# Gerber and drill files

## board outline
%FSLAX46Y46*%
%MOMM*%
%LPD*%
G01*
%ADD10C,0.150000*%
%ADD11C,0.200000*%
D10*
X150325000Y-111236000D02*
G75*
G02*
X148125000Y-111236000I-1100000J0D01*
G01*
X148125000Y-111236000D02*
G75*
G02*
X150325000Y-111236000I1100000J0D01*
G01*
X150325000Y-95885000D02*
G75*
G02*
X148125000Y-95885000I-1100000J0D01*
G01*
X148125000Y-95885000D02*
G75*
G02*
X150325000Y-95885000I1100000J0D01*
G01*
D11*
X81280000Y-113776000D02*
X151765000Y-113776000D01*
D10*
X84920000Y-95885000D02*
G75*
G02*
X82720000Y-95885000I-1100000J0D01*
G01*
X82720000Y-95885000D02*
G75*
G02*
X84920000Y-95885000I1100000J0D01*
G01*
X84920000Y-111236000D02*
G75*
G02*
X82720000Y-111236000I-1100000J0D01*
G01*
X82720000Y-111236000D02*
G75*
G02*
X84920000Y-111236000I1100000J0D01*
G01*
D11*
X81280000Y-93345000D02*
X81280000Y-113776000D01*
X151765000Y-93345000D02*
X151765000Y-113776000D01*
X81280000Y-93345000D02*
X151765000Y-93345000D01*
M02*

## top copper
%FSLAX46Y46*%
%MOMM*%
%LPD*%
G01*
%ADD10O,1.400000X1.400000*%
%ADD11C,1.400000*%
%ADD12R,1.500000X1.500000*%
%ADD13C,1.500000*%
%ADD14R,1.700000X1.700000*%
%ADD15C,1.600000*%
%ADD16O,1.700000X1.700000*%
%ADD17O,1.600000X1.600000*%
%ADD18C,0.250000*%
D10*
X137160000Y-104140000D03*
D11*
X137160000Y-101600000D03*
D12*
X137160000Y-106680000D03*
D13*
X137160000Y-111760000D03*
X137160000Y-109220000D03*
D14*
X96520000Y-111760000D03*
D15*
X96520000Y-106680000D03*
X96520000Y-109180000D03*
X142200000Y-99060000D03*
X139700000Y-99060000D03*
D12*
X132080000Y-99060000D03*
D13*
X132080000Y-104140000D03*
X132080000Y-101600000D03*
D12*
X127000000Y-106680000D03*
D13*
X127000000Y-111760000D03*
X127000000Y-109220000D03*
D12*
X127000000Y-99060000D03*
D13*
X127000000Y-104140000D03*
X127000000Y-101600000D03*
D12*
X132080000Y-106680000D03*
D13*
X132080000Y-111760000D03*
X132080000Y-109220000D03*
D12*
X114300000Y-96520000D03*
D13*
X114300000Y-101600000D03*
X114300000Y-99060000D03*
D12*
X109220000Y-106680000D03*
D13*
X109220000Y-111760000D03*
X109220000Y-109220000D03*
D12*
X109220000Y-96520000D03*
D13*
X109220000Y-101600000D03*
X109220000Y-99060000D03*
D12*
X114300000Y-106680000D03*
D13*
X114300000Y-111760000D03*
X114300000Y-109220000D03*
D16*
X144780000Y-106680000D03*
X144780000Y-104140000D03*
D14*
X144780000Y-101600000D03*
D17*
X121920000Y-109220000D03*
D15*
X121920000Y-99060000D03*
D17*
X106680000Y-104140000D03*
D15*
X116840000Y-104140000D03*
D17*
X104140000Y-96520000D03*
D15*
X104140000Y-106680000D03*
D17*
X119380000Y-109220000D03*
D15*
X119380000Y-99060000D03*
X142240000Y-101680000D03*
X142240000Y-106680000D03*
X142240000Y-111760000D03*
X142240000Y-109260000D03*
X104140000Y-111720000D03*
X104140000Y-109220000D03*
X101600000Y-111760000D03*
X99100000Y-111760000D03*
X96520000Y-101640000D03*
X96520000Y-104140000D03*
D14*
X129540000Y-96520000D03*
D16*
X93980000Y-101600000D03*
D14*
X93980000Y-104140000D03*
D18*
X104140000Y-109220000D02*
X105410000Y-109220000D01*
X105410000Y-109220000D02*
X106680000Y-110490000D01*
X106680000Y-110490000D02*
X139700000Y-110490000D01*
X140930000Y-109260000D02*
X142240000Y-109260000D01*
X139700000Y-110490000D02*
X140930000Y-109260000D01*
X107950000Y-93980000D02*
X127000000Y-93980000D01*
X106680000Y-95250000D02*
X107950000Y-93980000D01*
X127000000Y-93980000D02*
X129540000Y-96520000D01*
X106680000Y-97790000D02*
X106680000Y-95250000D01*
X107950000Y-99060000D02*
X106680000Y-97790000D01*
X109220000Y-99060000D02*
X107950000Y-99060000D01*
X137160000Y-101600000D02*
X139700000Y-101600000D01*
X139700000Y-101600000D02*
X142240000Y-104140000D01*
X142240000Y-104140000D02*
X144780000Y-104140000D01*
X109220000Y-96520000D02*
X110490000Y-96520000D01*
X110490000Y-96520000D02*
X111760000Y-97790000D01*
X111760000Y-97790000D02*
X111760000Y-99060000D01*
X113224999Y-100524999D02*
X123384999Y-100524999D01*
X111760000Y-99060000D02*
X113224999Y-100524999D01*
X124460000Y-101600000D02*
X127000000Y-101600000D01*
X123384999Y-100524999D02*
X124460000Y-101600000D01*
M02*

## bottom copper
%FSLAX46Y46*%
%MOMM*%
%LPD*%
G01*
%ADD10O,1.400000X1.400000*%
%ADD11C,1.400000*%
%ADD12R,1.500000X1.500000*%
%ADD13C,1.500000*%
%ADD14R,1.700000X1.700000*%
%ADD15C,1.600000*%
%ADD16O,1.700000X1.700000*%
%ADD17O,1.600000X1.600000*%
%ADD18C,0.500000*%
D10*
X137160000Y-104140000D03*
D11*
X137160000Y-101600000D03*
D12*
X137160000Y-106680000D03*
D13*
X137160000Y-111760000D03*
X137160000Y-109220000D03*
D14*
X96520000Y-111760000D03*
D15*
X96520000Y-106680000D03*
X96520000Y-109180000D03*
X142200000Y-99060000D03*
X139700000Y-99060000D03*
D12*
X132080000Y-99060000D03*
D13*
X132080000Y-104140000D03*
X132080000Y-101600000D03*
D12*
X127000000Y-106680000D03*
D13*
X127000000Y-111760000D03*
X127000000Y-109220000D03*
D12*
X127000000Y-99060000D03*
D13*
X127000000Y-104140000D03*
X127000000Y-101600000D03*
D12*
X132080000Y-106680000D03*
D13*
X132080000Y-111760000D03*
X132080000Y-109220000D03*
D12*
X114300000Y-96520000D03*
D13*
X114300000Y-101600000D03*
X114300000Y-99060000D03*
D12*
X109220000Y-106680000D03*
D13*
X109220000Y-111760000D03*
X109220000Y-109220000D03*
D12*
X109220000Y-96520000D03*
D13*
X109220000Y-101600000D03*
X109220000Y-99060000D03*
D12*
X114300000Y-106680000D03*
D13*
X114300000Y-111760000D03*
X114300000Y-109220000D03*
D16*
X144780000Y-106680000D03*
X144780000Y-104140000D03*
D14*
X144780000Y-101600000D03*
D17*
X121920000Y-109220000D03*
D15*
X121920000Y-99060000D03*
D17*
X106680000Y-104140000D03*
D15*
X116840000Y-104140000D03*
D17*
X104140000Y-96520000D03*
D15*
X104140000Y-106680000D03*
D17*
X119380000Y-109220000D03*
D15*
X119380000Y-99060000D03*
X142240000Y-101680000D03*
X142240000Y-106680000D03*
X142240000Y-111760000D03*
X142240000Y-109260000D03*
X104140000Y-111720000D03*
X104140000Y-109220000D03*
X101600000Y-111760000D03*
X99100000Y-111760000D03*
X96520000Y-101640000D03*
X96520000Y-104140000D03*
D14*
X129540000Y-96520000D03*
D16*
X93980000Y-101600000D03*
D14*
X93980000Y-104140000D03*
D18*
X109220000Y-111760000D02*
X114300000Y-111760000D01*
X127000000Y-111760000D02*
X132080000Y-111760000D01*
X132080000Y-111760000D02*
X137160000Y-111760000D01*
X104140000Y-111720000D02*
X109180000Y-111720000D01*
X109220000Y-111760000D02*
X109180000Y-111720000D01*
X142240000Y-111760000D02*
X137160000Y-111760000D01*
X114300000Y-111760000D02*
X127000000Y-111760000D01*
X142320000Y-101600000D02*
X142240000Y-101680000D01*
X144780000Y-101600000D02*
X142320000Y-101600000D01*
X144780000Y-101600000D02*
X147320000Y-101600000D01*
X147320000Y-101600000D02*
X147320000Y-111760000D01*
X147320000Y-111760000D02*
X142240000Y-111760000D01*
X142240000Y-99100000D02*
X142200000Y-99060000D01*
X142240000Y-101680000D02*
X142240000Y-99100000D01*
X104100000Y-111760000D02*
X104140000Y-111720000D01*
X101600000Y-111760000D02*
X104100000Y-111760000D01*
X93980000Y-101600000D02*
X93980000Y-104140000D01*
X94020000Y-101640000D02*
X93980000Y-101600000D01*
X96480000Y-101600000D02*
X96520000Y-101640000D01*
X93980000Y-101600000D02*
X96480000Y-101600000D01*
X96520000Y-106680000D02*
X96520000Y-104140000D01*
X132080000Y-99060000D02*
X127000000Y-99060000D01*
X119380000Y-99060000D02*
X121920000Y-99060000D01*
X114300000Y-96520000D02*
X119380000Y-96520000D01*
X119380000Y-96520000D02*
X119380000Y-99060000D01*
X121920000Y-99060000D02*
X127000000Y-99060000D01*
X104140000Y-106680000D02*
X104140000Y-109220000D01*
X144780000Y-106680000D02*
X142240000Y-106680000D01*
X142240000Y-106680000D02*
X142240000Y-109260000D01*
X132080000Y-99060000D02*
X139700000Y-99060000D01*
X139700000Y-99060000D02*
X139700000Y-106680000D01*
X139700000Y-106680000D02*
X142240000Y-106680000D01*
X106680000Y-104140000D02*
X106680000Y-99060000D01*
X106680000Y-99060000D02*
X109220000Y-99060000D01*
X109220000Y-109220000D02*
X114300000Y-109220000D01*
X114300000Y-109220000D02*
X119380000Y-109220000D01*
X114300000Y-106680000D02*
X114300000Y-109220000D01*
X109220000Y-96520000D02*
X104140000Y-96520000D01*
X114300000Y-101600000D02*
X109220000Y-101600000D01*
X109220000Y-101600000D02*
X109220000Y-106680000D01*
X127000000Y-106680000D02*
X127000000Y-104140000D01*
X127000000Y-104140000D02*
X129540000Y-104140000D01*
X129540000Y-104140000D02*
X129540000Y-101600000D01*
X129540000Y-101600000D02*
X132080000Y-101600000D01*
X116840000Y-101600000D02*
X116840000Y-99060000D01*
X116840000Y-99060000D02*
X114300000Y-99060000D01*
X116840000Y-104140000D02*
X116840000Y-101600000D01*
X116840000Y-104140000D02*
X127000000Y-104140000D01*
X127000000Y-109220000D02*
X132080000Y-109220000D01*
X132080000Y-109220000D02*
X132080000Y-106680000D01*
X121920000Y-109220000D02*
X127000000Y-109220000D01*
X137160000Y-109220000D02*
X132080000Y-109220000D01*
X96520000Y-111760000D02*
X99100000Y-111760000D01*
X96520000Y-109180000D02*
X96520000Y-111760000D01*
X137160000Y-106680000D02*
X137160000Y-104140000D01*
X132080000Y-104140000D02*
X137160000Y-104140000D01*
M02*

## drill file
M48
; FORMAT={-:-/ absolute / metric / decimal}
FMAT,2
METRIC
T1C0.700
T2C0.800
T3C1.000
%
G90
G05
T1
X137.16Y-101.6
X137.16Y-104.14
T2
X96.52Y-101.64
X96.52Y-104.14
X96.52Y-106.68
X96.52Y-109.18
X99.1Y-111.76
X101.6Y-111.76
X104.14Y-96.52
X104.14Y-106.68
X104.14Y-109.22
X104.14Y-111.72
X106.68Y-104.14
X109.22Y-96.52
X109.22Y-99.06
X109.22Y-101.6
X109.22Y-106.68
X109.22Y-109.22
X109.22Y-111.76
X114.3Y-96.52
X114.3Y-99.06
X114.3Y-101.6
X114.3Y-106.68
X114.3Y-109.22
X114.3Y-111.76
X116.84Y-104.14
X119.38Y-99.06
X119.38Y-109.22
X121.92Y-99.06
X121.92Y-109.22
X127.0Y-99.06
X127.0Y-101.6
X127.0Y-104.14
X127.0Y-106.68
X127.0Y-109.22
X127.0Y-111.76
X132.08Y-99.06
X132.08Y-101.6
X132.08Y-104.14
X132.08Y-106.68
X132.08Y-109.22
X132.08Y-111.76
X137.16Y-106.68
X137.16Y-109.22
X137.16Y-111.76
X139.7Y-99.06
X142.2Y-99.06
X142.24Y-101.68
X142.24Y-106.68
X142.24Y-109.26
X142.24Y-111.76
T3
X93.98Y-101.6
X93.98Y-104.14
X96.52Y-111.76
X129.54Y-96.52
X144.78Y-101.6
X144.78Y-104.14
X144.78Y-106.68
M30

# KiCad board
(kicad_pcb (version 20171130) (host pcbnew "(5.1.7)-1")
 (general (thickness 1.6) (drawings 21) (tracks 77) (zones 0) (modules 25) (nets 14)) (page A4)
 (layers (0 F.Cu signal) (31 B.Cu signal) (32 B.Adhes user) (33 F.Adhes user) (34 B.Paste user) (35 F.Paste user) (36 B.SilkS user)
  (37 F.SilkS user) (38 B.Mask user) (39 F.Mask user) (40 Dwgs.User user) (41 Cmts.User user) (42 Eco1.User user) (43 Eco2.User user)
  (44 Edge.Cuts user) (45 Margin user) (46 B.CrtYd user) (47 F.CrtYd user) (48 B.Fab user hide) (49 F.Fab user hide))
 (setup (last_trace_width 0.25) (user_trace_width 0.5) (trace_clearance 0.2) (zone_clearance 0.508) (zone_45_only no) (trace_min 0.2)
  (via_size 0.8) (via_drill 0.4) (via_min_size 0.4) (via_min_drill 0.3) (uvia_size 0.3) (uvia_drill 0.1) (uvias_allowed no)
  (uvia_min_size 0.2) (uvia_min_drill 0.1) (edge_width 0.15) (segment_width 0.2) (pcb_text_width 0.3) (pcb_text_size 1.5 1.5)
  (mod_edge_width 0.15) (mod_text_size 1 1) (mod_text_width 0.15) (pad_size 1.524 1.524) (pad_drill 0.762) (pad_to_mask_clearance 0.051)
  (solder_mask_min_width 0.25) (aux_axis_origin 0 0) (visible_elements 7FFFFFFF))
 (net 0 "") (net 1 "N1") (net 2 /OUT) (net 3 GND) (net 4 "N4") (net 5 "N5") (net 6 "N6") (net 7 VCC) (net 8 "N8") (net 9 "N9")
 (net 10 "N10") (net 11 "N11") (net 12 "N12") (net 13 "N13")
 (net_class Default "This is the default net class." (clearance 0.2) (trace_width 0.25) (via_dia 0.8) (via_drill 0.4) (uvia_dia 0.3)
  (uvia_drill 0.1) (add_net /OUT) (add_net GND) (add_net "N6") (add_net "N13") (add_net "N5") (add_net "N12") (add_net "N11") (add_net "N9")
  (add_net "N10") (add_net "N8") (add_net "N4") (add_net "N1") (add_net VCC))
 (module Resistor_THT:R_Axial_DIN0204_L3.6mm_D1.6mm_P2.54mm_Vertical (layer F.Cu) (at 137.16 101.6 270)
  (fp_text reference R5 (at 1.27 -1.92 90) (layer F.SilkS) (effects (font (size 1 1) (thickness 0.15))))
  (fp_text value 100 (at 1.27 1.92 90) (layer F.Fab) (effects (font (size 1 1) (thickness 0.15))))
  (pad 2 thru_hole oval (at 2.54 0 270) (size 1.4 1.4) (drill 0.7) (layers *.Cu *.Mask) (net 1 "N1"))
  (pad 1 thru_hole circle (at 0 0 270) (size 1.4 1.4) (drill 0.7) (layers *.Cu *.Mask) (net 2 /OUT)))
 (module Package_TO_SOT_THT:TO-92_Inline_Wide (layer F.Cu) (at 137.16 106.68 270)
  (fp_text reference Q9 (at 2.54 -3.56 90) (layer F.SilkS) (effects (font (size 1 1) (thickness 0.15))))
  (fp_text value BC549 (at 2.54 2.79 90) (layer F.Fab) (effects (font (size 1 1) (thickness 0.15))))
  (pad 1 thru_hole rect (at 0 0 270) (size 1.5 1.5) (drill 0.8) (layers *.Cu *.Mask) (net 1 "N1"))
  (pad 3 thru_hole circle (at 5.08 0 270) (size 1.5 1.5) (drill 0.8) (layers *.Cu *.Mask) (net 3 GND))
  (pad 2 thru_hole circle (at 2.54 0 270) (size 1.5 1.5) (drill 0.8) (layers *.Cu *.Mask) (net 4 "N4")))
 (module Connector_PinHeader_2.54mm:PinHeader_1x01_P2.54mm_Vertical (layer F.Cu) (at 96.52 111.76)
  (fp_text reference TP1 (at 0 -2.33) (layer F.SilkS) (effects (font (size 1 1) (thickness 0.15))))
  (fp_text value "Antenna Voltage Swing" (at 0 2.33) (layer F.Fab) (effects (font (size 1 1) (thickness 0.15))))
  (pad 1 thru_hole rect (at 0 0) (size 1.7 1.7) (drill 1) (layers *.Cu *.Mask) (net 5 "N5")))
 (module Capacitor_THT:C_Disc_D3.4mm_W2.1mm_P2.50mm (layer F.Cu) (at 96.52 109.18 90)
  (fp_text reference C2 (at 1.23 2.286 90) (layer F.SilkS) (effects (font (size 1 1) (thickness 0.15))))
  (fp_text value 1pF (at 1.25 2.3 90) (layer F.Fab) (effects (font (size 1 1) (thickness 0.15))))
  (pad 2 thru_hole circle (at 2.5 0 90) (size 1.6 1.6) (drill 0.8) (layers *.Cu *.Mask) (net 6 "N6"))
  (pad 1 thru_hole circle (at 0 0 90) (size 1.6 1.6) (drill 0.8) (layers *.Cu *.Mask) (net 5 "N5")))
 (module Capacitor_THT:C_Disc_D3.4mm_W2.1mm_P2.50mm (layer F.Cu) (at 139.7 99.06)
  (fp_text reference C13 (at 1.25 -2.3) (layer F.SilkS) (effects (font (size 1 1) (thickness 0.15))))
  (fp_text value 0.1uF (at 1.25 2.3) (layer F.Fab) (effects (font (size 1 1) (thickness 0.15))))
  (pad 2 thru_hole circle (at 2.5 0) (size 1.6 1.6) (drill 0.8) (layers *.Cu *.Mask) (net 3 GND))
  (pad 1 thru_hole circle (at 0 0) (size 1.6 1.6) (drill 0.8) (layers *.Cu *.Mask) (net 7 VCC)))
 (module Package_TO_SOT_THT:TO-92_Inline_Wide (layer F.Cu) (at 132.08 99.06 270)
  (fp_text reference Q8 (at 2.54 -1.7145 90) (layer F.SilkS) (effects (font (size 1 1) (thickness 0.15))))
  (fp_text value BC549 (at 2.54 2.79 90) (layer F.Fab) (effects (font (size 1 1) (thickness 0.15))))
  (pad 1 thru_hole rect (at 0 0 270) (size 1.5 1.5) (drill 0.8) (layers *.Cu *.Mask) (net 7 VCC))
  (pad 3 thru_hole circle (at 5.08 0 270) (size 1.5 1.5) (drill 0.8) (layers *.Cu *.Mask) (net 1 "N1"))
  (pad 2 thru_hole circle (at 2.54 0 270) (size 1.5 1.5) (drill 0.8) (layers *.Cu *.Mask) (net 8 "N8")))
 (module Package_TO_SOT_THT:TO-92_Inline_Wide (layer F.Cu) (at 127 106.68 270)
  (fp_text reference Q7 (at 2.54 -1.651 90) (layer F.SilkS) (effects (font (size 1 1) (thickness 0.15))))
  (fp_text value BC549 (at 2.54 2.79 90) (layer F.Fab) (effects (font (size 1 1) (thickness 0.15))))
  (pad 1 thru_hole rect (at 0 0 270) (size 1.5 1.5) (drill 0.8) (layers *.Cu *.Mask) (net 8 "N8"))
  (pad 3 thru_hole circle (at 5.08 0 270) (size 1.5 1.5) (drill 0.8) (layers *.Cu *.Mask) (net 3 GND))
  (pad 2 thru_hole circle (at 2.54 0 270) (size 1.5 1.5) (drill 0.8) (layers *.Cu *.Mask) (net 4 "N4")))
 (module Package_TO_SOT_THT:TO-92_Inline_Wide (layer F.Cu) (at 127 99.06 270)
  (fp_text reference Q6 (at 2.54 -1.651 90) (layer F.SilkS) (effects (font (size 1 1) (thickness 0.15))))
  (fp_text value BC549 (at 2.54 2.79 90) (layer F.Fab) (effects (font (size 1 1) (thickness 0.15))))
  (pad 1 thru_hole rect (at 0 0 270) (size 1.5 1.5) (drill 0.8) (layers *.Cu *.Mask) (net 7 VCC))
  (pad 3 thru_hole circle (at 5.08 0 270) (size 1.5 1.5) (drill 0.8) (layers *.Cu *.Mask) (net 8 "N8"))
  (pad 2 thru_hole circle (at 2.54 0 270) (size 1.5 1.5) (drill 0.8) (layers *.Cu *.Mask) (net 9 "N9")))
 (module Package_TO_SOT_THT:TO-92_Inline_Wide (layer F.Cu) (at 132.08 106.68 270)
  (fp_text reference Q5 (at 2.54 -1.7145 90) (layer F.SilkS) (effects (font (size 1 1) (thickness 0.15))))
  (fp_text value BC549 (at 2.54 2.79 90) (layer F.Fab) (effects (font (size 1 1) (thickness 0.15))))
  (pad 1 thru_hole rect (at 0 0 270) (size 1.5 1.5) (drill 0.8) (layers *.Cu *.Mask) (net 4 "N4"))
  (pad 3 thru_hole circle (at 5.08 0 270) (size 1.5 1.5) (drill 0.8) (layers *.Cu *.Mask) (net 3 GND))
  (pad 2 thru_hole circle (at 2.54 0 270) (size 1.5 1.5) (drill 0.8) (layers *.Cu *.Mask) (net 4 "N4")))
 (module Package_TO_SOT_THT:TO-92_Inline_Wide (layer F.Cu) (at 114.3 96.52 270)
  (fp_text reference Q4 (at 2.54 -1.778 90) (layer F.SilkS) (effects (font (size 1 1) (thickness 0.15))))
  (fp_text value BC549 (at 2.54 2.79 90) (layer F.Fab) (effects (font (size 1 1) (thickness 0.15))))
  (pad 1 thru_hole rect (at 0 0 270) (size 1.5 1.5) (drill 0.8) (layers *.Cu *.Mask) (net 7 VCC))
  (pad 3 thru_hole circle (at 5.08 0 270) (size 1.5 1.5) (drill 0.8) (layers *.Cu *.Mask) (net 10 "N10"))
  (pad 2 thru_hole circle (at 2.54 0 270) (size 1.5 1.5) (drill 0.8) (layers *.Cu *.Mask) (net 8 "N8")))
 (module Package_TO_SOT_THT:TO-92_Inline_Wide (layer F.Cu) (at 109.22 106.68 270)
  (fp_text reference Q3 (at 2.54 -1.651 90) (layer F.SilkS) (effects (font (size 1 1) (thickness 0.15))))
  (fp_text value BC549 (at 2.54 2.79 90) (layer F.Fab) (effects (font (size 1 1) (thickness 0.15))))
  (pad 1 thru_hole rect (at 0 0 270) (size 1.5 1.5) (drill 0.8) (layers *.Cu *.Mask) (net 10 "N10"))
  (pad 3 thru_hole circle (at 5.08 0 270) (size 1.5 1.5) (drill 0.8) (layers *.Cu *.Mask) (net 3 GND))
  (pad 2 thru_hole circle (at 2.54 0 270) (size 1.5 1.5) (drill 0.8) (layers *.Cu *.Mask) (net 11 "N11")))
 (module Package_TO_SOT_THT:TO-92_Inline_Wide (layer F.Cu) (at 109.22 96.52 270)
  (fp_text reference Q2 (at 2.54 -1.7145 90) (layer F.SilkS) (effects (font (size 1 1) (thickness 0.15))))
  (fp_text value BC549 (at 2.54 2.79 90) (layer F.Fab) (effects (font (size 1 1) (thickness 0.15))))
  (pad 1 thru_hole rect (at 0 0 270) (size 1.5 1.5) (drill 0.8) (layers *.Cu *.Mask) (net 9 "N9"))
  (pad 3 thru_hole circle (at 5.08 0 270) (size 1.5 1.5) (drill 0.8) (layers *.Cu *.Mask) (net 10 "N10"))
  (pad 2 thru_hole circle (at 2.54 0 270) (size 1.5 1.5) (drill 0.8) (layers *.Cu *.Mask) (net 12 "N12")))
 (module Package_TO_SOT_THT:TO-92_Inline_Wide (layer F.Cu) (at 114.3 106.68 270)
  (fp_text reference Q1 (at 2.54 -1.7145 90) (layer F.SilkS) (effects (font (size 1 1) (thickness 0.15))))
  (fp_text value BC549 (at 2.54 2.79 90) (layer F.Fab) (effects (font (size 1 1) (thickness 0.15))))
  (pad 1 thru_hole rect (at 0 0 270) (size 1.5 1.5) (drill 0.8) (layers *.Cu *.Mask) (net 11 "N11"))
  (pad 3 thru_hole circle (at 5.08 0 270) (size 1.5 1.5) (drill 0.8) (layers *.Cu *.Mask) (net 3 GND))
  (pad 2 thru_hole circle (at 2.54 0 270) (size 1.5 1.5) (drill 0.8) (layers *.Cu *.Mask) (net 11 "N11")))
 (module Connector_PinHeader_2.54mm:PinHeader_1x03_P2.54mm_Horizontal (layer F.Cu) (at 144.78 101.6)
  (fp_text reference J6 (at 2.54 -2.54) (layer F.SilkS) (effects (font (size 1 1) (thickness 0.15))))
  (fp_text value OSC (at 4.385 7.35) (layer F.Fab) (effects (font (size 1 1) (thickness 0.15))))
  (pad 3 thru_hole oval (at 0 5.08) (size 1.7 1.7) (drill 1) (layers *.Cu *.Mask) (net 7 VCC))
  (pad 2 thru_hole oval (at 0 2.54) (size 1.7 1.7) (drill 1) (layers *.Cu *.Mask) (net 2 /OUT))
  (pad 1 thru_hole rect (at 0 0) (size 1.7 1.7) (drill 1) (layers *.Cu *.Mask) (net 3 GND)))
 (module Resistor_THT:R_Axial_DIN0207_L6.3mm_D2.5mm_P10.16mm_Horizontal (layer F.Cu) (at 121.92 99.06 270)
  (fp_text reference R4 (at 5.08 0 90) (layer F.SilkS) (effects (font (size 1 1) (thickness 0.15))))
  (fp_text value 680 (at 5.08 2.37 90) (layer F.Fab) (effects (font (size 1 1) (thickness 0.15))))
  (pad 2 thru_hole oval (at 10.16 0 270) (size 1.6 1.6) (drill 0.8) (layers *.Cu *.Mask) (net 4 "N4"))
  (pad 1 thru_hole circle (at 0 0 270) (size 1.6 1.6) (drill 0.8) (layers *.Cu *.Mask) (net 7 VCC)))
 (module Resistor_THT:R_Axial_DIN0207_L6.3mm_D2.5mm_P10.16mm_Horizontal (layer F.Cu) (at 116.84 104.14 180)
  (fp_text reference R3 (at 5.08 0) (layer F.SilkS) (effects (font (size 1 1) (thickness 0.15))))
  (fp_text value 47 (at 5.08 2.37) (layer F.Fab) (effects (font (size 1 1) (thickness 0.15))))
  (pad 2 thru_hole oval (at 10.16 0 180) (size 1.6 1.6) (drill 0.8) (layers *.Cu *.Mask) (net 12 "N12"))
  (pad 1 thru_hole circle (at 0 0 180) (size 1.6 1.6) (drill 0.8) (layers *.Cu *.Mask) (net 8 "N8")))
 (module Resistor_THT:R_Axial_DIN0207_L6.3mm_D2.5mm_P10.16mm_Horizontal (layer F.Cu) (at 104.14 106.68 90)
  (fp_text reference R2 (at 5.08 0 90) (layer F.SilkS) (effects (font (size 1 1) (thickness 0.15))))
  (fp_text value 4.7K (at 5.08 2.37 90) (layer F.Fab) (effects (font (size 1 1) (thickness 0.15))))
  (pad 2 thru_hole oval (at 10.16 0 90) (size 1.6 1.6) (drill 0.8) (layers *.Cu *.Mask) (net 9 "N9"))
  (pad 1 thru_hole circle (at 0 0 90) (size 1.6 1.6) (drill 0.8) (layers *.Cu *.Mask) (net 7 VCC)))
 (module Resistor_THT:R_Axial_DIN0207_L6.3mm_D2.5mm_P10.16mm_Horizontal (layer F.Cu) (at 119.38 99.06 270)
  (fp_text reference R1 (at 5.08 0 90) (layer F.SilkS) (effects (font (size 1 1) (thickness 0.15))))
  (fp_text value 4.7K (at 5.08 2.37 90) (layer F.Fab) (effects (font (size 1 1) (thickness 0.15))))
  (pad 2 thru_hole oval (at 10.16 0 270) (size 1.6 1.6) (drill 0.8) (layers *.Cu *.Mask) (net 11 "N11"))
  (pad 1 thru_hole circle (at 0 0 270) (size 1.6 1.6) (drill 0.8) (layers *.Cu *.Mask) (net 7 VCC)))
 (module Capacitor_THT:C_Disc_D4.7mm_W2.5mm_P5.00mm (layer F.Cu) (at 142.24 106.68 90)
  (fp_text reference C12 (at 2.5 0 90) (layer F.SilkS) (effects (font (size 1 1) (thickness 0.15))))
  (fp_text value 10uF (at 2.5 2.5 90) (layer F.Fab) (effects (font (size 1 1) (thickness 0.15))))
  (pad 2 thru_hole circle (at 5 0 90) (size 1.6 1.6) (drill 0.8) (layers *.Cu *.Mask) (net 3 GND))
  (pad 1 thru_hole circle (at 0 0 90) (size 1.6 1.6) (drill 0.8) (layers *.Cu *.Mask) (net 7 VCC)))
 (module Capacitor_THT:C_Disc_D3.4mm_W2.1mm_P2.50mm (layer F.Cu) (at 142.24 109.26 270)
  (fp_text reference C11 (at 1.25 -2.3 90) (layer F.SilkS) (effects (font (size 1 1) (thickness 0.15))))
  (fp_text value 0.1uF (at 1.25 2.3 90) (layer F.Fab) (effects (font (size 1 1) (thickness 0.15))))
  (pad 2 thru_hole circle (at 2.5 0 270) (size 1.6 1.6) (drill 0.8) (layers *.Cu *.Mask) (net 3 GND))
  (pad 1 thru_hole circle (at 0 0 270) (size 1.6 1.6) (drill 0.8) (layers *.Cu *.Mask) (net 7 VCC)))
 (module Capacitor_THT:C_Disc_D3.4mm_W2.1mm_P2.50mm (layer F.Cu) (at 104.14 109.22 270)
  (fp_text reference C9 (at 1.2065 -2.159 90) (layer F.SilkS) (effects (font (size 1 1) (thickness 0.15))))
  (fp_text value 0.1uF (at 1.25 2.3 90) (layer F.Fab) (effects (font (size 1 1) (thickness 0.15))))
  (pad 2 thru_hole circle (at 2.5 0 270) (size 1.6 1.6) (drill 0.8) (layers *.Cu *.Mask) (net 3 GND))
  (pad 1 thru_hole circle (at 0 0 270) (size 1.6 1.6) (drill 0.8) (layers *.Cu *.Mask) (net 7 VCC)))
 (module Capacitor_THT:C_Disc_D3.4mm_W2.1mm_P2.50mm (layer F.Cu) (at 99.1 111.76)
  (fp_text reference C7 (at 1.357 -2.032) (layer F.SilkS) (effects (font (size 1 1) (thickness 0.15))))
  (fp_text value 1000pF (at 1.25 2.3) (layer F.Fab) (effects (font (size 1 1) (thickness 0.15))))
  (pad 2 thru_hole circle (at 2.5 0) (size 1.6 1.6) (drill 0.8) (layers *.Cu *.Mask) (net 3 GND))
  (pad 1 thru_hole circle (at 0 0) (size 1.6 1.6) (drill 0.8) (layers *.Cu *.Mask) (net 5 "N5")))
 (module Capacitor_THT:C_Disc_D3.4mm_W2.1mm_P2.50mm (layer F.Cu) (at 96.52 104.14 90)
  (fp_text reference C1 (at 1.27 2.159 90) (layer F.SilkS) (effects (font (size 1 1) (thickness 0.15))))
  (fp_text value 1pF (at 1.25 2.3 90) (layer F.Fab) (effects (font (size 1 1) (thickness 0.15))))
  (pad 2 thru_hole circle (at 2.5 0 90) (size 1.6 1.6) (drill 0.8) (layers *.Cu *.Mask) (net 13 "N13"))
  (pad 1 thru_hole circle (at 0 0 90) (size 1.6 1.6) (drill 0.8) (layers *.Cu *.Mask) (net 6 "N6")))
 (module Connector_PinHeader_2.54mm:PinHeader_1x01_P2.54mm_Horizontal (layer F.Cu) (at 129.54 96.52)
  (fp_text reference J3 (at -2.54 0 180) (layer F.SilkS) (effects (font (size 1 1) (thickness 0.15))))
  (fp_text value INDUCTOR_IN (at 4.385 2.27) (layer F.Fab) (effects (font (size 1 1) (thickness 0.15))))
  (pad 1 thru_hole rect (at 0 0) (size 1.7 1.7) (drill 1) (layers *.Cu *.Mask) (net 12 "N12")))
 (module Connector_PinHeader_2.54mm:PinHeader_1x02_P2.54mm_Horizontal (layer F.Cu) (at 93.98 104.14 180)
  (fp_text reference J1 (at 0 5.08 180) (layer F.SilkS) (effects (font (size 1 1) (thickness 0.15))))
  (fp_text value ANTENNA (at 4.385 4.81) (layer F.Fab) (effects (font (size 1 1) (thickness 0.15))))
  (pad 2 thru_hole oval (at 0 2.54 180) (size 1.7 1.7) (drill 1) (layers *.Cu *.Mask) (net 13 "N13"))
  (pad 1 thru_hole rect (at 0 0 180) (size 1.7 1.7) (drill 1) (layers *.Cu *.Mask) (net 13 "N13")))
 (gr_circle (center 149.225 111.236) (end 150.325 111.236) (layer Edge.Cuts) (width 0.15))
 (gr_circle (center 149.225 95.885) (end 150.325 95.885) (layer Edge.Cuts) (width 0.15))
 (gr_line (start 81.28 113.776) (end 151.765 113.776) (layer Edge.Cuts) (width 0.2))
 (gr_circle (center 83.82 95.885) (end 84.92 95.885) (layer Edge.Cuts) (width 0.15))
 (gr_circle (center 83.82 111.236) (end 84.92 111.236) (layer Edge.Cuts) (width 0.15))
 (gr_line (start 81.28 93.345) (end 81.28 113.776) (layer Edge.Cuts) (width 0.2))
 (gr_line (start 151.765 93.345) (end 151.765 113.776) (layer Edge.Cuts) (width 0.2))
 (gr_line (start 81.28 93.345) (end 151.765 93.345) (layer Edge.Cuts) (width 0.2))
 (segment (start 109.22 111.76) (end 114.3 111.76) (width 0.5) (layer B.Cu) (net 3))
 (segment (start 127 111.76) (end 132.08 111.76) (width 0.5) (layer B.Cu) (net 3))
 (segment (start 132.08 111.76) (end 137.16 111.76) (width 0.5) (layer B.Cu) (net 3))
 (segment (start 104.14 111.72) (end 109.18 111.72) (width 0.5) (layer B.Cu) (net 3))
 (segment (start 109.22 111.76) (end 109.18 111.72) (width 0.5) (layer B.Cu) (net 3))
 (segment (start 142.24 111.76) (end 137.16 111.76) (width 0.5) (layer B.Cu) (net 3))
 (segment (start 114.3 111.76) (end 127 111.76) (width 0.5) (layer B.Cu) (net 3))
 (segment (start 142.32 101.6) (end 142.24 101.68) (width 0.5) (layer B.Cu) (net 3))
 (segment (start 144.78 101.6) (end 142.32 101.6) (width 0.5) (layer B.Cu) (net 3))
 (segment (start 144.78 101.6) (end 147.32 101.6) (width 0.5) (layer B.Cu) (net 3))
 (segment (start 147.32 101.6) (end 147.32 111.76) (width 0.5) (layer B.Cu) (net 3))
 (segment (start 147.32 111.76) (end 142.24 111.76) (width 0.5) (layer B.Cu) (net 3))
 (segment (start 142.24 99.1) (end 142.2 99.06) (width 0.5) (layer B.Cu) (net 3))
 (segment (start 142.24 101.68) (end 142.24 99.1) (width 0.5) (layer B.Cu) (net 3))
 (segment (start 104.1 111.76) (end 104.14 111.72) (width 0.5) (layer B.Cu) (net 3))
 (segment (start 101.6 111.76) (end 104.1 111.76) (width 0.5) (layer B.Cu) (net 3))
 (segment (start 93.98 101.6) (end 93.98 104.14) (width 0.5) (layer B.Cu) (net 13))
 (segment (start 94.02 101.64) (end 93.98 101.6) (width 0.5) (layer B.Cu) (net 13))
 (segment (start 96.48 101.6) (end 96.52 101.64) (width 0.5) (layer B.Cu) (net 13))
 (segment (start 93.98 101.6) (end 96.48 101.6) (width 0.5) (layer B.Cu) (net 13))
 (segment (start 96.52 106.68) (end 96.52 104.14) (width 0.5) (layer B.Cu) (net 6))
 (segment (start 132.08 99.06) (end 127 99.06) (width 0.5) (layer B.Cu) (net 7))
 (segment (start 119.38 99.06) (end 121.92 99.06) (width 0.5) (layer B.Cu) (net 7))
 (segment (start 114.3 96.52) (end 119.38 96.52) (width 0.5) (layer B.Cu) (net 7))
 (segment (start 119.38 96.52) (end 119.38 99.06) (width 0.5) (layer B.Cu) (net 7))
 (segment (start 121.92 99.06) (end 127 99.06) (width 0.5) (layer B.Cu) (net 7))
 (segment (start 104.14 106.68) (end 104.14 109.22) (width 0.5) (layer B.Cu) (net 7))
 (segment (start 144.78 106.68) (end 142.24 106.68) (width 0.5) (layer B.Cu) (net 7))
 (segment (start 142.24 106.68) (end 142.24 109.26) (width 0.5) (layer B.Cu) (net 7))
 (segment (start 132.08 99.06) (end 139.7 99.06) (width 0.5) (layer B.Cu) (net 7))
 (segment (start 139.7 99.06) (end 139.7 106.68) (width 0.5) (layer B.Cu) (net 7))
 (segment (start 139.7 106.68) (end 142.24 106.68) (width 0.5) (layer B.Cu) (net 7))
 (segment (start 104.14 109.22) (end 105.41 109.22) (width 0.25) (layer F.Cu) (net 7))
 (segment (start 105.41 109.22) (end 106.68 110.49) (width 0.25) (layer F.Cu) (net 7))
 (segment (start 106.68 110.49) (end 139.7 110.49) (width 0.25) (layer F.Cu) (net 7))
 (segment (start 140.93 109.26) (end 142.24 109.26) (width 0.25) (layer F.Cu) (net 7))
 (segment (start 139.7 110.49) (end 140.93 109.26) (width 0.25) (layer F.Cu) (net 7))
 (segment (start 106.68 104.14) (end 106.68 99.06) (width 0.5) (layer B.Cu) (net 12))
 (segment (start 106.68 99.06) (end 109.22 99.06) (width 0.5) (layer B.Cu) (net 12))
 (segment (start 107.95 93.98) (end 127 93.98) (width 0.25) (layer F.Cu) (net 12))
 (segment (start 106.68 95.25) (end 107.95 93.98) (width 0.25) (layer F.Cu) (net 12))
 (segment (start 127 93.98) (end 129.54 96.52) (width 0.25) (layer F.Cu) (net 12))
 (segment (start 106.68 97.79) (end 106.68 95.25) (width 0.25) (layer F.Cu) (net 12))
 (segment (start 107.95 99.06) (end 106.68 97.79) (width 0.25) (layer F.Cu) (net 12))
 (segment (start 109.22 99.06) (end 107.95 99.06) (width 0.25) (layer F.Cu) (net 12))
 (segment (start 137.16 101.6) (end 139.7 101.6) (width 0.25) (layer F.Cu) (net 2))
 (segment (start 139.7 101.6) (end 142.24 104.14) (width 0.25) (layer F.Cu) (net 2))
 (segment (start 142.24 104.14) (end 144.78 104.14) (width 0.25) (layer F.Cu) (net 2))
 (segment (start 109.22 109.22) (end 114.3 109.22) (width 0.5) (layer B.Cu) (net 11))
 (segment (start 114.3 109.22) (end 119.38 109.22) (width 0.5) (layer B.Cu) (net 11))
 (segment (start 114.3 106.68) (end 114.3 109.22) (width 0.5) (layer B.Cu) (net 11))
 (segment (start 109.22 96.52) (end 104.14 96.52) (width 0.5) (layer B.Cu) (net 9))
 (segment (start 109.22 96.52) (end 110.49 96.52) (width 0.25) (layer F.Cu) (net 9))
 (segment (start 110.49 96.52) (end 111.76 97.79) (width 0.25) (layer F.Cu) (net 9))
 (segment (start 111.76 97.79) (end 111.76 99.06) (width 0.25) (layer F.Cu) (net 9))
 (segment (start 113.224999 100.524999) (end 123.384999 100.524999) (width 0.25) (layer F.Cu) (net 9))
 (segment (start 111.76 99.06) (end 113.224999 100.524999) (width 0.25) (layer F.Cu) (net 9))
 (segment (start 124.46 101.6) (end 127 101.6) (width 0.25) (layer F.Cu) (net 9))
 (segment (start 123.384999 100.524999) (end 124.46 101.6) (width 0.25) (layer F.Cu) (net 9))
 (segment (start 114.3 101.6) (end 109.22 101.6) (width 0.5) (layer B.Cu) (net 10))
 (segment (start 109.22 101.6) (end 109.22 106.68) (width 0.5) (layer B.Cu) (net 10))
 (segment (start 127 106.68) (end 127 104.14) (width 0.5) (layer B.Cu) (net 8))
 (segment (start 127 104.14) (end 129.54 104.14) (width 0.5) (layer B.Cu) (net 8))
 (segment (start 129.54 104.14) (end 129.54 101.6) (width 0.5) (layer B.Cu) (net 8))
 (segment (start 129.54 101.6) (end 132.08 101.6) (width 0.5) (layer B.Cu) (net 8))
 (segment (start 116.84 101.6) (end 116.84 99.06) (width 0.5) (layer B.Cu) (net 8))
 (segment (start 116.84 99.06) (end 114.3 99.06) (width 0.5) (layer B.Cu) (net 8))
 (segment (start 116.84 104.14) (end 116.84 101.6) (width 0.5) (layer B.Cu) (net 8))
 (segment (start 116.84 104.14) (end 127 104.14) (width 0.5) (layer B.Cu) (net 8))
 (segment (start 127 109.22) (end 132.08 109.22) (width 0.5) (layer B.Cu) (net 4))
 (segment (start 132.08 109.22) (end 132.08 106.68) (width 0.5) (layer B.Cu) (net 4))
 (segment (start 121.92 109.22) (end 127 109.22) (width 0.5) (layer B.Cu) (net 4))
 (segment (start 137.16 109.22) (end 132.08 109.22) (width 0.5) (layer B.Cu) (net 4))
 (segment (start 96.52 111.76) (end 99.1 111.76) (width 0.5) (layer B.Cu) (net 5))
 (segment (start 96.52 109.18) (end 96.52 111.76) (width 0.5) (layer B.Cu) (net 5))
 (segment (start 137.16 106.68) (end 137.16 104.14) (width 0.5) (layer B.Cu) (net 1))
 (segment (start 132.08 104.14) (end 137.16 104.14) (width 0.5) (layer B.Cu) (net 1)))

